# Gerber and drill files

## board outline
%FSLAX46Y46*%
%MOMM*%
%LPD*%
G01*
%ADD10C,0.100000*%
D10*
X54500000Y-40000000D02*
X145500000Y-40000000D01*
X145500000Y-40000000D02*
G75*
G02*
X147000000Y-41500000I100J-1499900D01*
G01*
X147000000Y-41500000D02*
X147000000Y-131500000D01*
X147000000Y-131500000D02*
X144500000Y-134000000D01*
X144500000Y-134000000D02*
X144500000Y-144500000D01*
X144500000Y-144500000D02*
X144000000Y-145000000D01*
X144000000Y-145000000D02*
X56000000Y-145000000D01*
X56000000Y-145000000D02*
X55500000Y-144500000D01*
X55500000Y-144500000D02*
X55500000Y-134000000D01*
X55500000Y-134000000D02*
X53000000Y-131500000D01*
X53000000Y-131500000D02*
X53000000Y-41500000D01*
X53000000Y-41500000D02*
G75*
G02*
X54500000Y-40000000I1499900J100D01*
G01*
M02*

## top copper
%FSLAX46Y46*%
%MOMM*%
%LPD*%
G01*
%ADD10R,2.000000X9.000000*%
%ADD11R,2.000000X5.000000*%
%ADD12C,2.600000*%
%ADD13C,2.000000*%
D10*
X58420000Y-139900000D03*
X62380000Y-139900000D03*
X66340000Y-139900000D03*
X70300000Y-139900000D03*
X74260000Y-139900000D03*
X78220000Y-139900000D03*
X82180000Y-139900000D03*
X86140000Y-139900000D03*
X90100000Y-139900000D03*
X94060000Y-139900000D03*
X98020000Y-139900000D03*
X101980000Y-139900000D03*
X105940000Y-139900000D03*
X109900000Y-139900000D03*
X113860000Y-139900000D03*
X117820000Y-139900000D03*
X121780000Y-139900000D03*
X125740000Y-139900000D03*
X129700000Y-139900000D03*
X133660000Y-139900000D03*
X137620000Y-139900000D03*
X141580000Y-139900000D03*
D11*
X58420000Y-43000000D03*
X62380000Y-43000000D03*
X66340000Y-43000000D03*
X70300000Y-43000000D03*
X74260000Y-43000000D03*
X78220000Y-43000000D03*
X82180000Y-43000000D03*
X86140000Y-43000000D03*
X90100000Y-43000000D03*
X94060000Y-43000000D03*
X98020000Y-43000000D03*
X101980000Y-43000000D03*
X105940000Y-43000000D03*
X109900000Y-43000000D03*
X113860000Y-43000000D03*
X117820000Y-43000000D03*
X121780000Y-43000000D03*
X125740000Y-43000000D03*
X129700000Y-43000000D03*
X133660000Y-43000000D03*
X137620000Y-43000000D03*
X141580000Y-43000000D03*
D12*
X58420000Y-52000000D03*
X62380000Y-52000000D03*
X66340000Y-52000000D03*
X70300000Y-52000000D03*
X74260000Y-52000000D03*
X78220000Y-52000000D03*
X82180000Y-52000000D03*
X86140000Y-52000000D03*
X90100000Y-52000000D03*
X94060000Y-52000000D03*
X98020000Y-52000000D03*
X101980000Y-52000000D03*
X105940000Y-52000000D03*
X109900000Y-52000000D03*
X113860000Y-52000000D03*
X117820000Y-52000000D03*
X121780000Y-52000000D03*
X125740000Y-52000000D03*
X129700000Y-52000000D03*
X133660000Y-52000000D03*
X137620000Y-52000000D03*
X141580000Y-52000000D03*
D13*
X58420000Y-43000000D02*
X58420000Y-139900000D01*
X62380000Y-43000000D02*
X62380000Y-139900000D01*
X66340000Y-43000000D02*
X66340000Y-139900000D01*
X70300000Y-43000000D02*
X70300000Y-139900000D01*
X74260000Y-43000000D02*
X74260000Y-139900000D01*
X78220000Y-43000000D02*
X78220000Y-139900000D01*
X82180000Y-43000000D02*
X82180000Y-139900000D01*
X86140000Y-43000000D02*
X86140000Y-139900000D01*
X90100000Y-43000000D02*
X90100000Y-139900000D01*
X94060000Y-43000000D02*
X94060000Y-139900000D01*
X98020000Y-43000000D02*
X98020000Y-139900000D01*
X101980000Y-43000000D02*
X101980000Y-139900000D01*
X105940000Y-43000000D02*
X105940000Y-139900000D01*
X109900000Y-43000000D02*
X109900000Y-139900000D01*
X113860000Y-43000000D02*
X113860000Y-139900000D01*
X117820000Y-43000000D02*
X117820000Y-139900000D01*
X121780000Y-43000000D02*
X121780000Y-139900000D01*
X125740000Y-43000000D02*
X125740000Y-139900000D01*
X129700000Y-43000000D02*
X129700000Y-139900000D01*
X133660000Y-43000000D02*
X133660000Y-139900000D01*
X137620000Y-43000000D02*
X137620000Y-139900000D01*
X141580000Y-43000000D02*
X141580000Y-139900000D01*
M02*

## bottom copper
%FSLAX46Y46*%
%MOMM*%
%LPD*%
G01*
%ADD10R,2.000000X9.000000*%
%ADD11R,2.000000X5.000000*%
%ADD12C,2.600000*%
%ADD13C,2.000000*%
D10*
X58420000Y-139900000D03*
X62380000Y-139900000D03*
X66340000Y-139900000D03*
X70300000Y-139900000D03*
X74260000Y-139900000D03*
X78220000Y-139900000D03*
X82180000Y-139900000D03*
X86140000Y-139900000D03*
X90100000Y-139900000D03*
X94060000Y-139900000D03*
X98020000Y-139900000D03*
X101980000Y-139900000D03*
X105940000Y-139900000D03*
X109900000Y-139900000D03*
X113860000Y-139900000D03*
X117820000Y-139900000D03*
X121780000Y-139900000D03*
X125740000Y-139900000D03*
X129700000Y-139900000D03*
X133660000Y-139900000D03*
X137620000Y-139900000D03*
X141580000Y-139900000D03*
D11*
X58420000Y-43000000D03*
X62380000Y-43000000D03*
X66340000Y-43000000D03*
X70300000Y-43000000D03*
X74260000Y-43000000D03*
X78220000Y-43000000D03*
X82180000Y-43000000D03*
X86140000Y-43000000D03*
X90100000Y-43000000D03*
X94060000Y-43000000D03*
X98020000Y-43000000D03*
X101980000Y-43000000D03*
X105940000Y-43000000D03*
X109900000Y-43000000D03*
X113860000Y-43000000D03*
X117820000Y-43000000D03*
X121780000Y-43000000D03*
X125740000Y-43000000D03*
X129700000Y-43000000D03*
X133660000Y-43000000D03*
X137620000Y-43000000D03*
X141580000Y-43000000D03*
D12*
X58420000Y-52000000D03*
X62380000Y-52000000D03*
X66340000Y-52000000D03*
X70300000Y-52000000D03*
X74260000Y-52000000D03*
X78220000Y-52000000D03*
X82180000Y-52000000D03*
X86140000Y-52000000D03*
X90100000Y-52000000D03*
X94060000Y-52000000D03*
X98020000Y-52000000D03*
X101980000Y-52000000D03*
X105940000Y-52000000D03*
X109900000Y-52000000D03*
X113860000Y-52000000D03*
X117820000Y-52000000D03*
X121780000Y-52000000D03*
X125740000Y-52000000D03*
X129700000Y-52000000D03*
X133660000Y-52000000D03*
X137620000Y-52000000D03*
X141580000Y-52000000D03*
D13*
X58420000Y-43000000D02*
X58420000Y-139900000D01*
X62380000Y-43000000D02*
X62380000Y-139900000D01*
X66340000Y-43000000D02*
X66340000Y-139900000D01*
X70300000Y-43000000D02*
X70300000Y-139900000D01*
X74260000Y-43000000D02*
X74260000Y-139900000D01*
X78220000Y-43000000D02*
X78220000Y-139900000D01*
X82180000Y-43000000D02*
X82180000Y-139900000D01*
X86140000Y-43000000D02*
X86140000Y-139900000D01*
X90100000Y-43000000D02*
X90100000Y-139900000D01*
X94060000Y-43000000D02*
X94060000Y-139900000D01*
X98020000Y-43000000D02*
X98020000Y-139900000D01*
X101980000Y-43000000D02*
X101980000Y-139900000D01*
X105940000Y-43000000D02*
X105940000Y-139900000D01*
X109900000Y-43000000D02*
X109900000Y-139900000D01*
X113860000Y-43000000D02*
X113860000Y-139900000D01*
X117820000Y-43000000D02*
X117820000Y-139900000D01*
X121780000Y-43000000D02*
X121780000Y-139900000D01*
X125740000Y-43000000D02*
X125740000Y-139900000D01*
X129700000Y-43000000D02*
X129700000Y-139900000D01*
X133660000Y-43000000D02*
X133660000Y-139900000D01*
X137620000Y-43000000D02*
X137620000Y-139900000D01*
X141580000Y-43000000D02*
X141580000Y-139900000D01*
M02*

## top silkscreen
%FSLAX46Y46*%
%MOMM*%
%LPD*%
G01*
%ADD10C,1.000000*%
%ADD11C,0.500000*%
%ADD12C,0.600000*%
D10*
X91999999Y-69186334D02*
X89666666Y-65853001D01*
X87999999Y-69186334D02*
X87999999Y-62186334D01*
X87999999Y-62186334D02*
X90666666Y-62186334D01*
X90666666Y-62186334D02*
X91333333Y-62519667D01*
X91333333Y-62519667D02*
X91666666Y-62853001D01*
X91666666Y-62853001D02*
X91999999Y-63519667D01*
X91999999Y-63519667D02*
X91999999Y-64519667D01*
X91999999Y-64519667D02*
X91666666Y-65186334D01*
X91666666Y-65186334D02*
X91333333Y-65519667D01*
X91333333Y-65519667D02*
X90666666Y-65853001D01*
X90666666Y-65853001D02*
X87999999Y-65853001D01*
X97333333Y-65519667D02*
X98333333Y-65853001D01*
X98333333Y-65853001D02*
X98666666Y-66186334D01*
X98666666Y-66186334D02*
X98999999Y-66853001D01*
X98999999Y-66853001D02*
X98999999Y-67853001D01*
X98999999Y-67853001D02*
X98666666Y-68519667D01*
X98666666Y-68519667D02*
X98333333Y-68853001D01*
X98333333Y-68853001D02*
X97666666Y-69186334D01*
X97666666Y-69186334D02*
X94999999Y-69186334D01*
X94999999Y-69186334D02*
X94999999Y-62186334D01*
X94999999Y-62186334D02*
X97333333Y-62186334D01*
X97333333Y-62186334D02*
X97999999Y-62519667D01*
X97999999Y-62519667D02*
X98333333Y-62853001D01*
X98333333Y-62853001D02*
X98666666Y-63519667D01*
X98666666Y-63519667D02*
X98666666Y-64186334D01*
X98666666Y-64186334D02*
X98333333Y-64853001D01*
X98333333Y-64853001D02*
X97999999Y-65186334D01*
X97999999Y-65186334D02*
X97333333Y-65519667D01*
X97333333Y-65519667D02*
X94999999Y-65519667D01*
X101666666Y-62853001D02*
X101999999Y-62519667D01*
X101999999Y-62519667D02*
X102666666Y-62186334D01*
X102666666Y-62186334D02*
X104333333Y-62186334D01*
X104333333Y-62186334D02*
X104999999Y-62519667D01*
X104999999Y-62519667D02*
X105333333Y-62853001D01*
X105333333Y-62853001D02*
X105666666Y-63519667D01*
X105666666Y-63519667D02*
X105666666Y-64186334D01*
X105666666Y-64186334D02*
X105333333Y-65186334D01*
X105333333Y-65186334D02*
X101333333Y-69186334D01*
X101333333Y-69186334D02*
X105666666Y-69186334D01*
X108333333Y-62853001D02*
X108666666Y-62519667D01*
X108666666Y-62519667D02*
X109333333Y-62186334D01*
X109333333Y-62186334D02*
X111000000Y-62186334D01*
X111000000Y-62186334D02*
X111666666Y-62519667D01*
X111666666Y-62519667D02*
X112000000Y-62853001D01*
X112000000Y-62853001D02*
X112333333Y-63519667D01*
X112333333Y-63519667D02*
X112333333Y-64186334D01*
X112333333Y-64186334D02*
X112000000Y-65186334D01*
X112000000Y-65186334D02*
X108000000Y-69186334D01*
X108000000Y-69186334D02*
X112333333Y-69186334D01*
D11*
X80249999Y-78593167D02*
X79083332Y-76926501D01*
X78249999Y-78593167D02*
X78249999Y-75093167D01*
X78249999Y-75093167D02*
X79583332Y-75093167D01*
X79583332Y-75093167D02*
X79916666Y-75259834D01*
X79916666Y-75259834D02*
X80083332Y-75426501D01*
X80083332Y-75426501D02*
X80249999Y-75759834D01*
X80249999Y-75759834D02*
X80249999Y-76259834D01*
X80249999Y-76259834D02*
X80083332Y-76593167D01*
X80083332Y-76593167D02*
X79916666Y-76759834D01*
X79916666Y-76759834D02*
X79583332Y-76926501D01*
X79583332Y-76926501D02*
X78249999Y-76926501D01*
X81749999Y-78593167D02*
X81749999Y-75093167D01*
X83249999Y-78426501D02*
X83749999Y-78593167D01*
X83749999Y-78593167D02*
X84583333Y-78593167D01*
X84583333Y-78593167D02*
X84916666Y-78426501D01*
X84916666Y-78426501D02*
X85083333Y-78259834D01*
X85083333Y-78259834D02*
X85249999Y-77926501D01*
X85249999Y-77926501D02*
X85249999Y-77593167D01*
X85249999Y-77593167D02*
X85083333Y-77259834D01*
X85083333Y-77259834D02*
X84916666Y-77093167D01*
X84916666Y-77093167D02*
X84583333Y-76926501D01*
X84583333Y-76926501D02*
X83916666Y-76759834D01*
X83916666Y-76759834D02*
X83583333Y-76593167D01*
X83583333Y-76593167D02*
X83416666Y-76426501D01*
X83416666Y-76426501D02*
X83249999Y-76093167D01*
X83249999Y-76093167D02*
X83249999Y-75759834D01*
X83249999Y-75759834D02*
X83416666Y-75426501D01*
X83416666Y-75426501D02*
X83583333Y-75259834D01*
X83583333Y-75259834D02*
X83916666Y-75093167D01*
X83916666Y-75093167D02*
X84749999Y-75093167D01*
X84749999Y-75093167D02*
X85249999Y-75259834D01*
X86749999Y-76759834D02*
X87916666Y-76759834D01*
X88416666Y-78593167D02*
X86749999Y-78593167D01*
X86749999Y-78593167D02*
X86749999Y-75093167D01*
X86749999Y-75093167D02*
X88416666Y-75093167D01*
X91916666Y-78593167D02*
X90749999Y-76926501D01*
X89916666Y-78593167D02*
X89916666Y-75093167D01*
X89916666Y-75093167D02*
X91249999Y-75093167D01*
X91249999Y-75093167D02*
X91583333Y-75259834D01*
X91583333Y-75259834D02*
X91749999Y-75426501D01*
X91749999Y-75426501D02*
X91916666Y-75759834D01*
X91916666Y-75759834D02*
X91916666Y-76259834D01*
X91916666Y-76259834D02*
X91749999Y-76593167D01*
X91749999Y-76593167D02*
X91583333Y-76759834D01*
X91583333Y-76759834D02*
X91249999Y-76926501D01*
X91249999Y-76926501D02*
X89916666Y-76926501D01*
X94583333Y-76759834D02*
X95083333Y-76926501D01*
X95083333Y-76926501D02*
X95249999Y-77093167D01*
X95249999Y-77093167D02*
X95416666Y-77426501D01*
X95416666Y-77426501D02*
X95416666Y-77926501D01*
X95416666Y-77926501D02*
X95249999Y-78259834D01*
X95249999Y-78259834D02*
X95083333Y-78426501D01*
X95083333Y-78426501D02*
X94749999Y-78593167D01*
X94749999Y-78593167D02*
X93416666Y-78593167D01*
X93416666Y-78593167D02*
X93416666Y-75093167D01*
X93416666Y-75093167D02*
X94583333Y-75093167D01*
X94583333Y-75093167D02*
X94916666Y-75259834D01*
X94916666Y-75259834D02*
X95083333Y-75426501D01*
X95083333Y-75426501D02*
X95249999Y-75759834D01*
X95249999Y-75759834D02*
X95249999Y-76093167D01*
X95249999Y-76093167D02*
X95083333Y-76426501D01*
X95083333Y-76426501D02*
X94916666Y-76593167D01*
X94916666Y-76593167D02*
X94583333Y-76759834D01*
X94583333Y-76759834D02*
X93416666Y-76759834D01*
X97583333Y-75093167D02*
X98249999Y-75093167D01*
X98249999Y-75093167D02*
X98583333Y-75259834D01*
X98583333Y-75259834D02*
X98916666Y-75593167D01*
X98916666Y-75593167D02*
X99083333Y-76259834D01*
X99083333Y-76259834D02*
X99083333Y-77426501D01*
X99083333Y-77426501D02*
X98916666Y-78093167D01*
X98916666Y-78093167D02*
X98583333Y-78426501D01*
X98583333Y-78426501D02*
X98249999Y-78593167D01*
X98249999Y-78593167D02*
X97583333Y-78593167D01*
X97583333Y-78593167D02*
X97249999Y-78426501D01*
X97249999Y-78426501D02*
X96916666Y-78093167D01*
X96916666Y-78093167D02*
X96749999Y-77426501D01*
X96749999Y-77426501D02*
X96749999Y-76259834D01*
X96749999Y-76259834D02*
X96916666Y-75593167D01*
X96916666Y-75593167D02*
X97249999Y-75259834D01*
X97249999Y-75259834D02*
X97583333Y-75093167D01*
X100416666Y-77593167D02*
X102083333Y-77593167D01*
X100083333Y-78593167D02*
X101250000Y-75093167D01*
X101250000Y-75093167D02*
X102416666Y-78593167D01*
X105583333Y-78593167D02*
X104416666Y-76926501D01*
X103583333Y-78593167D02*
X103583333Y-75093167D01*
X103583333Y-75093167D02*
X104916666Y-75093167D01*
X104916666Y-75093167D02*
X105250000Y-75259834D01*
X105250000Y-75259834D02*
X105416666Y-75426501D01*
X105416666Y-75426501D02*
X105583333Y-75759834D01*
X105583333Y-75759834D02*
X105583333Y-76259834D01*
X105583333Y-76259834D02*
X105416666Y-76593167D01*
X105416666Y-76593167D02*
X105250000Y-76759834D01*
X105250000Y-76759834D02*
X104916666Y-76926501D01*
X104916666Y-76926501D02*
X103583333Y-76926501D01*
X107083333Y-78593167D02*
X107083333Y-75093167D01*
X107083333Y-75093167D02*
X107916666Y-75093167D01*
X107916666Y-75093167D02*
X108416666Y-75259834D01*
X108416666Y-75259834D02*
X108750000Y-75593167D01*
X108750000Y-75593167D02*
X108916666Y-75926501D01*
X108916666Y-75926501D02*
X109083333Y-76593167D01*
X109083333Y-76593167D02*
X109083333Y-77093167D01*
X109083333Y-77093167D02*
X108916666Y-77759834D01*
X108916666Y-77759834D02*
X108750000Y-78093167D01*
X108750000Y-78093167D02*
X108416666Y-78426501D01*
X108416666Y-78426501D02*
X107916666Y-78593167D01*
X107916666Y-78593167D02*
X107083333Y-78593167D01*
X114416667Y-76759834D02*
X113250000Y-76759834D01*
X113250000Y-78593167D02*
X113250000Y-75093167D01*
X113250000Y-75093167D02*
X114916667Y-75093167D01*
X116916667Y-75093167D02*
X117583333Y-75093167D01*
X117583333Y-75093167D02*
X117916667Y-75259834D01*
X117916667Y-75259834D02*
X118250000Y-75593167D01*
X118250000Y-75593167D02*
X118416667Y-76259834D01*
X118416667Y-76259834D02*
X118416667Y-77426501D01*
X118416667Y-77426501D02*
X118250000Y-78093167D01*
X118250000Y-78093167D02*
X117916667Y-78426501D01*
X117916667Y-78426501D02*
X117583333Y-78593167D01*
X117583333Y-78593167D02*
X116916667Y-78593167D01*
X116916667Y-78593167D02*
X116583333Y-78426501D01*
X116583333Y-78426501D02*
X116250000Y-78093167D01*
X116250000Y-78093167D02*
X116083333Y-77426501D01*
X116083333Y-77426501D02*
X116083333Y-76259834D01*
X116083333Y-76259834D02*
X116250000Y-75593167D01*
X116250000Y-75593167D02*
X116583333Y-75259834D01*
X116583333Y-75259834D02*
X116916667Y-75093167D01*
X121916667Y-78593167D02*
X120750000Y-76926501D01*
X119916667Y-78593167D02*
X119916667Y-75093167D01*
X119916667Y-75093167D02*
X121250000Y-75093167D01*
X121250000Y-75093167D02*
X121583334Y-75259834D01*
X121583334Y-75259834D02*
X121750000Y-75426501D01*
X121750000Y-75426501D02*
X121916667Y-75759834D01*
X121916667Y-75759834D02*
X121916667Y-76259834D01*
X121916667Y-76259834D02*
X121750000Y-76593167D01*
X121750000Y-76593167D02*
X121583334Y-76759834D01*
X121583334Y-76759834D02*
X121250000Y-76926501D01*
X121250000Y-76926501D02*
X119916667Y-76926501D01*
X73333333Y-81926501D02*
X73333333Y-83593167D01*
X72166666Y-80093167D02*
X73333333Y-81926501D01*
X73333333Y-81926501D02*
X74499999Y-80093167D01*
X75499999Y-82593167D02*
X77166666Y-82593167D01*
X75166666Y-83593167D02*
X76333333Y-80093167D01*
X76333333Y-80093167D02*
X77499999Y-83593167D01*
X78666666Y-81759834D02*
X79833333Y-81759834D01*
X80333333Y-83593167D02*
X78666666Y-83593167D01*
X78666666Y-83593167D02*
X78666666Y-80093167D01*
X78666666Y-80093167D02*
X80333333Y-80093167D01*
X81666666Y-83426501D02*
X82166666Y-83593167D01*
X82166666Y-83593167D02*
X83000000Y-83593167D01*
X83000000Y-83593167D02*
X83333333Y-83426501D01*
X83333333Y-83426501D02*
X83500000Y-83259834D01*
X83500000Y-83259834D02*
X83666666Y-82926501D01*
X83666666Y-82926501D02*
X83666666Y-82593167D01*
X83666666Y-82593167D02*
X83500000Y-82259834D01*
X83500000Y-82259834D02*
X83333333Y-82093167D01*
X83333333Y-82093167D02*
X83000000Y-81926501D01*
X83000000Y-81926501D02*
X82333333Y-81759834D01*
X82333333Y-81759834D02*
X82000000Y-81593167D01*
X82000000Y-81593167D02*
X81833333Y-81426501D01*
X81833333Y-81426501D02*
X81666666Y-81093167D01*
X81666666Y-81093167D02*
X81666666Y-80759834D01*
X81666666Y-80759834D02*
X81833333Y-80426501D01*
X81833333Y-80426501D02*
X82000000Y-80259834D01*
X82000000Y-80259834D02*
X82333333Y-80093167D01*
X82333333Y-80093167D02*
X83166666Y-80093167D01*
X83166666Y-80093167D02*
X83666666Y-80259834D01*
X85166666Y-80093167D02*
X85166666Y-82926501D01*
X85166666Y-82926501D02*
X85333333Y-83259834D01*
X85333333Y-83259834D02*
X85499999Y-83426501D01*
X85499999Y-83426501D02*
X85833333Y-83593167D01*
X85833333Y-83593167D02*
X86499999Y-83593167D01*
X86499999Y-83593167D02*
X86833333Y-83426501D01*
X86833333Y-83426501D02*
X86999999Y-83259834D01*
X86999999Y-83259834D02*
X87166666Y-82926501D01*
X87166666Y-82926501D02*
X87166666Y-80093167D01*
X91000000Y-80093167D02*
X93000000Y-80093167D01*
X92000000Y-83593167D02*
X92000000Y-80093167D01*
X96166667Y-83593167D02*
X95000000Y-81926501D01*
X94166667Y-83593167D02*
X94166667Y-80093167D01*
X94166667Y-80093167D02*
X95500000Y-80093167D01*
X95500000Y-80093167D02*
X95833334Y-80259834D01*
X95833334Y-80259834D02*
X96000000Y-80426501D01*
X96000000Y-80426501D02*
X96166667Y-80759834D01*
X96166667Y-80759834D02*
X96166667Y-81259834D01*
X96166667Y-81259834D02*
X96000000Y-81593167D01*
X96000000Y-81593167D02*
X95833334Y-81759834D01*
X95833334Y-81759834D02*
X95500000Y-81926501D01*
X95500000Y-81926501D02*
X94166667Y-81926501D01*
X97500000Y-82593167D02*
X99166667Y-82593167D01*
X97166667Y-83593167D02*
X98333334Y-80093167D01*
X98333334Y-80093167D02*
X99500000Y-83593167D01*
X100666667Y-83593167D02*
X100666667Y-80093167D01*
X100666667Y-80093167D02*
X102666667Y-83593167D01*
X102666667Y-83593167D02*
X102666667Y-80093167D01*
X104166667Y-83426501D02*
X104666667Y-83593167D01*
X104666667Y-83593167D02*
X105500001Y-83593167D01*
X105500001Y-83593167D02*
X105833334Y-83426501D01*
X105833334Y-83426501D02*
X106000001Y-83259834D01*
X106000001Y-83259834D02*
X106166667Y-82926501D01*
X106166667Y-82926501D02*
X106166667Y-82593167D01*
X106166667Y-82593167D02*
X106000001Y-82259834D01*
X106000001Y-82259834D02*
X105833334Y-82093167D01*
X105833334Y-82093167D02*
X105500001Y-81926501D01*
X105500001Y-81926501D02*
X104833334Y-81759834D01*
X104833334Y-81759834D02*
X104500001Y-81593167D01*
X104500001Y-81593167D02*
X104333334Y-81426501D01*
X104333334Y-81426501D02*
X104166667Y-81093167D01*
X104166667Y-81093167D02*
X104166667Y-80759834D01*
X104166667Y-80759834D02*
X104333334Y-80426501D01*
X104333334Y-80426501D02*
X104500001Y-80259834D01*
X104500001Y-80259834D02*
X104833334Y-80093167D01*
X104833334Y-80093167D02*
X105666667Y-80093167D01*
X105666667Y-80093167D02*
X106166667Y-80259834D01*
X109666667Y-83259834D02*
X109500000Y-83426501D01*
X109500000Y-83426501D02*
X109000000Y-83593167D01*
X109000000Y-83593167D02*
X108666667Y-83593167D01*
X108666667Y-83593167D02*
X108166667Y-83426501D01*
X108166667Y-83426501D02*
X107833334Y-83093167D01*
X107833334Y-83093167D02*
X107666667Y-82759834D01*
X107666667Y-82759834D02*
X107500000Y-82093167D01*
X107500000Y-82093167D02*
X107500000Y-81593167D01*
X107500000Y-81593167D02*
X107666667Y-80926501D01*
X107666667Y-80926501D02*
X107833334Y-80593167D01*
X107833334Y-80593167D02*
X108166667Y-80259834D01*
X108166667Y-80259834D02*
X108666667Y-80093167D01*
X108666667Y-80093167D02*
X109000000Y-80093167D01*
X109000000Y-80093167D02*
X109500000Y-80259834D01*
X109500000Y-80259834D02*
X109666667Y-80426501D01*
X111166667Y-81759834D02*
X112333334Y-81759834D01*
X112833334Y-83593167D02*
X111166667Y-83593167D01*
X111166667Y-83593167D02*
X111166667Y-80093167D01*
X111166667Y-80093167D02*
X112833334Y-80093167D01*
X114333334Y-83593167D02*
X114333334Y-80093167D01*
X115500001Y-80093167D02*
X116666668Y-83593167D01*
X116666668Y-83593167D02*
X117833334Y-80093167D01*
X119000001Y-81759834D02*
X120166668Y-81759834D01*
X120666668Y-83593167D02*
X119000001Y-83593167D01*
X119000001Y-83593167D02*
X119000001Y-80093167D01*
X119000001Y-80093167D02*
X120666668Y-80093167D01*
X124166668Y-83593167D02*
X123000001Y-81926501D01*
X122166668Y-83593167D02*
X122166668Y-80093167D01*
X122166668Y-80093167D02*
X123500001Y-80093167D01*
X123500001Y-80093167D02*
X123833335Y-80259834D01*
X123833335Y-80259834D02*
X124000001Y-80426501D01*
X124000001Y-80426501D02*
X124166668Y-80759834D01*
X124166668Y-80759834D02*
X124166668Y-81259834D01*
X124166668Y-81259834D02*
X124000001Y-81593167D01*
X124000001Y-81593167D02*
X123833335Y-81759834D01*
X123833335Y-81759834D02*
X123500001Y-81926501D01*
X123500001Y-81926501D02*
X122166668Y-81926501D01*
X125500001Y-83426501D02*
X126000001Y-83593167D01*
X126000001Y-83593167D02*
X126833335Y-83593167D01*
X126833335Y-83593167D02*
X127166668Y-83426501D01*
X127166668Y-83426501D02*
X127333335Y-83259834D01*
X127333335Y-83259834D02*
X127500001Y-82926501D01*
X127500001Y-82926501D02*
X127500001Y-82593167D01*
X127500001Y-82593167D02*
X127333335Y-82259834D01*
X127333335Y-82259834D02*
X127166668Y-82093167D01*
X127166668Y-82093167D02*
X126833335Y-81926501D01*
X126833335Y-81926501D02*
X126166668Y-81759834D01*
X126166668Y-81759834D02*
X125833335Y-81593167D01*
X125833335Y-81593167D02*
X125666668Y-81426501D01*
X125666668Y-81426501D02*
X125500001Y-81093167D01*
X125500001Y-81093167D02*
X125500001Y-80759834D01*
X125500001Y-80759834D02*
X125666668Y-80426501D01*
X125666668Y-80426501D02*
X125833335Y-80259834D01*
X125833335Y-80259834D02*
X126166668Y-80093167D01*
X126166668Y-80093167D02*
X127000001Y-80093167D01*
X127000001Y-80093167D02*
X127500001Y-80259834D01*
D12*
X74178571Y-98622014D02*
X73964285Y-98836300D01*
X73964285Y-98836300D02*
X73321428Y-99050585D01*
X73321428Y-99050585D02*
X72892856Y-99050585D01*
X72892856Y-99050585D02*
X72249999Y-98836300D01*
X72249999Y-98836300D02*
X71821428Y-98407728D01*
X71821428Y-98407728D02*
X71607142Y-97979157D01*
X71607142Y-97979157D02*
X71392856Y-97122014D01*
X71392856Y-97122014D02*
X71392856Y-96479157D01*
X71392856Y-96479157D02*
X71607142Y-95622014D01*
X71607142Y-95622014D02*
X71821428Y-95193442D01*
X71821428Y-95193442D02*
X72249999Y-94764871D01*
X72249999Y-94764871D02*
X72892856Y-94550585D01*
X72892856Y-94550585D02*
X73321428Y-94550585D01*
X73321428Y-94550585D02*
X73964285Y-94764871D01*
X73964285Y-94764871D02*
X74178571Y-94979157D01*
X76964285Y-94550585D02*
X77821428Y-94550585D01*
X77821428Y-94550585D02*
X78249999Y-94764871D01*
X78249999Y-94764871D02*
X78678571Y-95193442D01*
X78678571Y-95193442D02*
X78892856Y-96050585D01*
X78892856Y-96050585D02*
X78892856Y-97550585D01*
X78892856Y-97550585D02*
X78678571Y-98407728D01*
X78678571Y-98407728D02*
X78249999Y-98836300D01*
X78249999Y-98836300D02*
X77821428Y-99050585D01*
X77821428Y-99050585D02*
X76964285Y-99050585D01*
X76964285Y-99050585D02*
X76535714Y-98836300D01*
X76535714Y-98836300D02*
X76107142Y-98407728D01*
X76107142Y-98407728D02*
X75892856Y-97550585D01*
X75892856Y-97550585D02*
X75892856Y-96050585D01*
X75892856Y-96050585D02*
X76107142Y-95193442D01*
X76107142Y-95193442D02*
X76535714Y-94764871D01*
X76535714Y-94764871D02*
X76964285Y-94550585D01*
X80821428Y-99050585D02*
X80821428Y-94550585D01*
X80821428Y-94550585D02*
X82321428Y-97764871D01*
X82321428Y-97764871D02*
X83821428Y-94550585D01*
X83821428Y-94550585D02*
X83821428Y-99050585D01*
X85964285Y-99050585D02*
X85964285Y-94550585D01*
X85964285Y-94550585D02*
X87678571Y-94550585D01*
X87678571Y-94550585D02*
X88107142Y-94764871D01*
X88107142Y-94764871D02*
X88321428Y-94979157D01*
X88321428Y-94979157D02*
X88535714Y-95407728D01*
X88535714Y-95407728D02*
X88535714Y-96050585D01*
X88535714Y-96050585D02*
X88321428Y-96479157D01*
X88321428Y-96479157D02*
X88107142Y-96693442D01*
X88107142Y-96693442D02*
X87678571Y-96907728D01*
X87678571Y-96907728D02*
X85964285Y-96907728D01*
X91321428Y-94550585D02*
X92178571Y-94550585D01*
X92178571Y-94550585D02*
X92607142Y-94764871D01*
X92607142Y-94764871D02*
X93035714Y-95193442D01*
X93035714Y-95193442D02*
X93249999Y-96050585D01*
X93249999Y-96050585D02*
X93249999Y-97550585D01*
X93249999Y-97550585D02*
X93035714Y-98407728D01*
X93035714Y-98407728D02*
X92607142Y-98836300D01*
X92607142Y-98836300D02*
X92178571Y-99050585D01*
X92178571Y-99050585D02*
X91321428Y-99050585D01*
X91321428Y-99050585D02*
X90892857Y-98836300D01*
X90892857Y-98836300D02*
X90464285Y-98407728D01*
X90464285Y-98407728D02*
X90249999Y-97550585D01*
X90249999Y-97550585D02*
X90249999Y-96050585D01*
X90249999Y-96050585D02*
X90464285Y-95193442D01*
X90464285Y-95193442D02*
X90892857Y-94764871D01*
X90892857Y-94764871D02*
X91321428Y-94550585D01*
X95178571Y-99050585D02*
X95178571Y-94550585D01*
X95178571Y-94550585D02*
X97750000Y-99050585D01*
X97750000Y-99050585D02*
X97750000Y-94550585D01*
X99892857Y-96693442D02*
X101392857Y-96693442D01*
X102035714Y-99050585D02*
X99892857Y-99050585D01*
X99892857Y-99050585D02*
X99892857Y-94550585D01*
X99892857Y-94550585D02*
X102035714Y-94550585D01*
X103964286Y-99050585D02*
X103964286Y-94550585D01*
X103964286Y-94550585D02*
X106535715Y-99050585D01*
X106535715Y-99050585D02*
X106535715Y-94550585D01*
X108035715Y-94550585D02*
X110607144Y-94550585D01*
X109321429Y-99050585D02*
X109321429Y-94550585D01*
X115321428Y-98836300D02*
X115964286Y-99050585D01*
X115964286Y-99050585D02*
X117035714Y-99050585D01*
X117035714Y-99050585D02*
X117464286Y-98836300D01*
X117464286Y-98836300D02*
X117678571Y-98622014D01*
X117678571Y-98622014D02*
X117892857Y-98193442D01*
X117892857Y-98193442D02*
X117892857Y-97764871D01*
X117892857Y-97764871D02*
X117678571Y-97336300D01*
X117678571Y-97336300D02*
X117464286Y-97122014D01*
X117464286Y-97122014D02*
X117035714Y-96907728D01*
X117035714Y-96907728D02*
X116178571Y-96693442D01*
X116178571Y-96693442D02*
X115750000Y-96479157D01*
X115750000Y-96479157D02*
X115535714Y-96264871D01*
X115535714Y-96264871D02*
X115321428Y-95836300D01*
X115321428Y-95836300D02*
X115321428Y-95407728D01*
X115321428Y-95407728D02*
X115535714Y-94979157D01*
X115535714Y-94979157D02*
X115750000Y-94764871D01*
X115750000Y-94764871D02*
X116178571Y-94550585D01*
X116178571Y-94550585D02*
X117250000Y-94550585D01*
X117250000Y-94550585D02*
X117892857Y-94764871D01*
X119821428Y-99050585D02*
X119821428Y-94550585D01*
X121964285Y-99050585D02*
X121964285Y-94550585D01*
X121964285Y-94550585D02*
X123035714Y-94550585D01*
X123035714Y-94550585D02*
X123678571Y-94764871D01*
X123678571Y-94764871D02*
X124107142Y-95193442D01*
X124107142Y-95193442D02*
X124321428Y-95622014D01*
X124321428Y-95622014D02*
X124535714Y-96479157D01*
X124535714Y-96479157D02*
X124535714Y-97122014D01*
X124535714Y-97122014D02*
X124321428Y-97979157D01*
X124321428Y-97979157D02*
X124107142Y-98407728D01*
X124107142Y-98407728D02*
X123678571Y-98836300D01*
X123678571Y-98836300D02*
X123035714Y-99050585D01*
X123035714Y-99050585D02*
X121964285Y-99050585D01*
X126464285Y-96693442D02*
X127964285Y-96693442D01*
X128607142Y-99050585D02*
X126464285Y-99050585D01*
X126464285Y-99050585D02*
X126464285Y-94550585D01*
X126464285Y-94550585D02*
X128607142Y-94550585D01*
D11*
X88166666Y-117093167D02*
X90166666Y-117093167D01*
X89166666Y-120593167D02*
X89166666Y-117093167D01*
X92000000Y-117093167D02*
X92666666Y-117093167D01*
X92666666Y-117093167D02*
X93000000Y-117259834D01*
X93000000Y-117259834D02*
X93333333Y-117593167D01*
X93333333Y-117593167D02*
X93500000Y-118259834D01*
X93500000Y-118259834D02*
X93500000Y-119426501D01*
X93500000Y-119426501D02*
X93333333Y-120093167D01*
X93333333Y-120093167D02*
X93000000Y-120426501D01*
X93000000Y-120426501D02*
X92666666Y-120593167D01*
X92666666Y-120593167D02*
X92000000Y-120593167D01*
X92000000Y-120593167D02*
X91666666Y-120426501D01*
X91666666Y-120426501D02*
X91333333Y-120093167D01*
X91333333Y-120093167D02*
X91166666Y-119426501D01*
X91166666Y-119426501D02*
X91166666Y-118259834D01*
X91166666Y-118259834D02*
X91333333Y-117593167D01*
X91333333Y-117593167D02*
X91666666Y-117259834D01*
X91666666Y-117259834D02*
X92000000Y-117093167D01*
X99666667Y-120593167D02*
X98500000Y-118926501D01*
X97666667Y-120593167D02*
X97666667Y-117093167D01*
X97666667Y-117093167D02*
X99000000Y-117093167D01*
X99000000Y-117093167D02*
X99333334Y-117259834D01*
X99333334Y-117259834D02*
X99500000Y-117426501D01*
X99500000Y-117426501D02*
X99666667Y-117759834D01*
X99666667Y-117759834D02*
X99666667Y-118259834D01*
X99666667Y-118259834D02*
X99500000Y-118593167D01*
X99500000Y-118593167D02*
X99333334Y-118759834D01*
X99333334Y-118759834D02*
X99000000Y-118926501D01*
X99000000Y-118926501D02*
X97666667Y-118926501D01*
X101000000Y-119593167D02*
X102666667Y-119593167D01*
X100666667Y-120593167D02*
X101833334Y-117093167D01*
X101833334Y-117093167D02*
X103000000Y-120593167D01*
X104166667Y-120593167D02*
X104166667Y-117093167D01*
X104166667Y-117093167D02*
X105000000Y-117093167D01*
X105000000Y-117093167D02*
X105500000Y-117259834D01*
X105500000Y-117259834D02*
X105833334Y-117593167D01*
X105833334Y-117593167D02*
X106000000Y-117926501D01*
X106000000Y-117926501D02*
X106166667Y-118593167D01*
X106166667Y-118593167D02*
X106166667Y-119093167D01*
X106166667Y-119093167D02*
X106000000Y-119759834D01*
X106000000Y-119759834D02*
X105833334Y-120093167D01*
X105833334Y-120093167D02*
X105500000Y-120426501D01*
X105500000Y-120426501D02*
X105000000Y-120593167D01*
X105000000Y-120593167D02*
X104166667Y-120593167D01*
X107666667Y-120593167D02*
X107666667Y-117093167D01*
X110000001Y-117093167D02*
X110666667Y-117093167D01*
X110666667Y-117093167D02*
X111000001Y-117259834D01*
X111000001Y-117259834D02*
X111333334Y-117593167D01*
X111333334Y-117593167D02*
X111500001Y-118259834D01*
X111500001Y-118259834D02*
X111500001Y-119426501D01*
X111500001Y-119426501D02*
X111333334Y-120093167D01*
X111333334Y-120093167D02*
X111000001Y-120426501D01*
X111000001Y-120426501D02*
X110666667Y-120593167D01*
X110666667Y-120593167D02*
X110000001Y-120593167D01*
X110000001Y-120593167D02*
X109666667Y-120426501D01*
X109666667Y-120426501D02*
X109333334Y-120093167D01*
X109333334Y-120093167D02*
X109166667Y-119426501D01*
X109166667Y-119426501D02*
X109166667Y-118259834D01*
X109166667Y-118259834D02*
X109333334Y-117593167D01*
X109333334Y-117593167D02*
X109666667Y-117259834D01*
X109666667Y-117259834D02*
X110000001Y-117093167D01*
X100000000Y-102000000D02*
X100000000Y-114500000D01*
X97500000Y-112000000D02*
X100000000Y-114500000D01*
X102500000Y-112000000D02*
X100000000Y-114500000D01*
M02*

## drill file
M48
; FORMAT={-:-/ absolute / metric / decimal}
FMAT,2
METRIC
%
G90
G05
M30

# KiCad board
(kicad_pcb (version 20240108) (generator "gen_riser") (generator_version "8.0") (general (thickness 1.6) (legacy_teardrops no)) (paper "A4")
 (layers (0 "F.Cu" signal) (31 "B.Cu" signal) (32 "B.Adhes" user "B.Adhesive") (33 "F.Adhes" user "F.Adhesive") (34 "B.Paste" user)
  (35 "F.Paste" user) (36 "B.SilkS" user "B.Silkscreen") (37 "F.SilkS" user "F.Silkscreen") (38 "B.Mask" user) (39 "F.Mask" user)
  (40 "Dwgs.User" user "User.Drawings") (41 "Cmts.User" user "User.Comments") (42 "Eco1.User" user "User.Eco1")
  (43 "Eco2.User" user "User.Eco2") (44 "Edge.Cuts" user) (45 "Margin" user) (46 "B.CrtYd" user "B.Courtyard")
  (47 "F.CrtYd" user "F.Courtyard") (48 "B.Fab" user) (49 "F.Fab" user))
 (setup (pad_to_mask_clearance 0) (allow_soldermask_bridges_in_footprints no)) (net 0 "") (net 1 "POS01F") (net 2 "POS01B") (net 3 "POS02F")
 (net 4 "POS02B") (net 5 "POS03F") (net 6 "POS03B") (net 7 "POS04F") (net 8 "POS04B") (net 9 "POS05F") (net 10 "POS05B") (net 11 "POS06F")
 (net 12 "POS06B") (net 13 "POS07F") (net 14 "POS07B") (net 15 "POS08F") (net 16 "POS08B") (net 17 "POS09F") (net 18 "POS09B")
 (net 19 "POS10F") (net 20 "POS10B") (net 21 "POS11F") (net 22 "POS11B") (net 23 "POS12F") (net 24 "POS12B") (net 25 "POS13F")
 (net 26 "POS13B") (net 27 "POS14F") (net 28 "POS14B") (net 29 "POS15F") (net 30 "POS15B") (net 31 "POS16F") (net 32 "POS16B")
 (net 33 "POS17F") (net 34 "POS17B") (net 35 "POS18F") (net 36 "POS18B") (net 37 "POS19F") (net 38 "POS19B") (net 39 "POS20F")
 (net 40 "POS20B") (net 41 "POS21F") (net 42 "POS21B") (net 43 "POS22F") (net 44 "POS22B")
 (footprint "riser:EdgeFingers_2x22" (layer "F.Cu") (at 100 40)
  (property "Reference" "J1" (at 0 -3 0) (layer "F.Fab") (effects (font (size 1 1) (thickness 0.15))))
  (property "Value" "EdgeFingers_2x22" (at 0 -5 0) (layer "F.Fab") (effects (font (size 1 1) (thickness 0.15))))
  (pad "1" smd rect (at -41.58 99.9) (size 2 9) (layers "F.Cu" "F.Mask") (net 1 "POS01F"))
  (pad "1B" smd rect (at -41.58 99.9) (size 2 9) (layers "B.Cu" "B.Mask") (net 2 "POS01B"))
  (pad "2" smd rect (at -37.62 99.9) (size 2 9) (layers "F.Cu" "F.Mask") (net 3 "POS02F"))
  (pad "2B" smd rect (at -37.62 99.9) (size 2 9) (layers "B.Cu" "B.Mask") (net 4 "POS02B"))
  (pad "3" smd rect (at -33.66 99.9) (size 2 9) (layers "F.Cu" "F.Mask") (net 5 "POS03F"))
  (pad "3B" smd rect (at -33.66 99.9) (size 2 9) (layers "B.Cu" "B.Mask") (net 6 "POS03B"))
  (pad "4" smd rect (at -29.7 99.9) (size 2 9) (layers "F.Cu" "F.Mask") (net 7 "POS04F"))
  (pad "4B" smd rect (at -29.7 99.9) (size 2 9) (layers "B.Cu" "B.Mask") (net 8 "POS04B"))
  (pad "5" smd rect (at -25.74 99.9) (size 2 9) (layers "F.Cu" "F.Mask") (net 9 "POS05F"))
  (pad "5B" smd rect (at -25.74 99.9) (size 2 9) (layers "B.Cu" "B.Mask") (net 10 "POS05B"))
  (pad "6" smd rect (at -21.78 99.9) (size 2 9) (layers "F.Cu" "F.Mask") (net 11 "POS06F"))
  (pad "6B" smd rect (at -21.78 99.9) (size 2 9) (layers "B.Cu" "B.Mask") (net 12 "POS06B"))
  (pad "7" smd rect (at -17.82 99.9) (size 2 9) (layers "F.Cu" "F.Mask") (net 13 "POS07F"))
  (pad "7B" smd rect (at -17.82 99.9) (size 2 9) (layers "B.Cu" "B.Mask") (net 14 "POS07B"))
  (pad "8" smd rect (at -13.86 99.9) (size 2 9) (layers "F.Cu" "F.Mask") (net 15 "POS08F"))
  (pad "8B" smd rect (at -13.86 99.9) (size 2 9) (layers "B.Cu" "B.Mask") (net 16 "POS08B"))
  (pad "9" smd rect (at -9.9 99.9) (size 2 9) (layers "F.Cu" "F.Mask") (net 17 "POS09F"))
  (pad "9B" smd rect (at -9.9 99.9) (size 2 9) (layers "B.Cu" "B.Mask") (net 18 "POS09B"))
  (pad "10" smd rect (at -5.94 99.9) (size 2 9) (layers "F.Cu" "F.Mask") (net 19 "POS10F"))
  (pad "10B" smd rect (at -5.94 99.9) (size 2 9) (layers "B.Cu" "B.Mask") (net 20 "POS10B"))
  (pad "11" smd rect (at -1.98 99.9) (size 2 9) (layers "F.Cu" "F.Mask") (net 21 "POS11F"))
  (pad "11B" smd rect (at -1.98 99.9) (size 2 9) (layers "B.Cu" "B.Mask") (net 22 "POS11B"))
  (pad "12" smd rect (at 1.98 99.9) (size 2 9) (layers "F.Cu" "F.Mask") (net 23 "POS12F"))
  (pad "12B" smd rect (at 1.98 99.9) (size 2 9) (layers "B.Cu" "B.Mask") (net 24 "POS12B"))
  (pad "13" smd rect (at 5.94 99.9) (size 2 9) (layers "F.Cu" "F.Mask") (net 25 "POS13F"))
  (pad "13B" smd rect (at 5.94 99.9) (size 2 9) (layers "B.Cu" "B.Mask") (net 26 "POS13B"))
  (pad "14" smd rect (at 9.9 99.9) (size 2 9) (layers "F.Cu" "F.Mask") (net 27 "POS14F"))
  (pad "14B" smd rect (at 9.9 99.9) (size 2 9) (layers "B.Cu" "B.Mask") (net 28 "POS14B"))
  (pad "15" smd rect (at 13.86 99.9) (size 2 9) (layers "F.Cu" "F.Mask") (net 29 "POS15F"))
  (pad "15B" smd rect (at 13.86 99.9) (size 2 9) (layers "B.Cu" "B.Mask") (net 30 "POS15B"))
  (pad "16" smd rect (at 17.82 99.9) (size 2 9) (layers "F.Cu" "F.Mask") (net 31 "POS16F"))
  (pad "16B" smd rect (at 17.82 99.9) (size 2 9) (layers "B.Cu" "B.Mask") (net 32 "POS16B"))
  (pad "17" smd rect (at 21.78 99.9) (size 2 9) (layers "F.Cu" "F.Mask") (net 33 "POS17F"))
  (pad "17B" smd rect (at 21.78 99.9) (size 2 9) (layers "B.Cu" "B.Mask") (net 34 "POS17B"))
  (pad "18" smd rect (at 25.74 99.9) (size 2 9) (layers "F.Cu" "F.Mask") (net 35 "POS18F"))
  (pad "18B" smd rect (at 25.74 99.9) (size 2 9) (layers "B.Cu" "B.Mask") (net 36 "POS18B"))
  (pad "19" smd rect (at 29.7 99.9) (size 2 9) (layers "F.Cu" "F.Mask") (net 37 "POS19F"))
  (pad "19B" smd rect (at 29.7 99.9) (size 2 9) (layers "B.Cu" "B.Mask") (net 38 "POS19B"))
  (pad "20" smd rect (at 33.66 99.9) (size 2 9) (layers "F.Cu" "F.Mask") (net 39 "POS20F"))
  (pad "20B" smd rect (at 33.66 99.9) (size 2 9) (layers "B.Cu" "B.Mask") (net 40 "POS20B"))
  (pad "21" smd rect (at 37.62 99.9) (size 2 9) (layers "F.Cu" "F.Mask") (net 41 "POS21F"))
  (pad "21B" smd rect (at 37.62 99.9) (size 2 9) (layers "B.Cu" "B.Mask") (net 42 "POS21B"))
  (pad "22" smd rect (at 41.58 99.9) (size 2 9) (layers "F.Cu" "F.Mask") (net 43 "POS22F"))
  (pad "22B" smd rect (at 41.58 99.9) (size 2 9) (layers "B.Cu" "B.Mask") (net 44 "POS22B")))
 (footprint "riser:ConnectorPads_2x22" (layer "F.Cu") (at 100 40)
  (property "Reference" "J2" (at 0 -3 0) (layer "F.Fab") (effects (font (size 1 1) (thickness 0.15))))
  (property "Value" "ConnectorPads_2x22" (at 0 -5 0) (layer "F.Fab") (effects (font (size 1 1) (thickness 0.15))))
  (pad "1" smd rect (at -41.58 3) (size 2 5) (layers "F.Cu" "F.Mask") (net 1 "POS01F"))
  (pad "1B" smd rect (at -41.58 3) (size 2 5) (layers "B.Cu" "B.Mask") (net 2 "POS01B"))
  (pad "2" smd rect (at -37.62 3) (size 2 5) (layers "F.Cu" "F.Mask") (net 3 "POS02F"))
  (pad "2B" smd rect (at -37.62 3) (size 2 5) (layers "B.Cu" "B.Mask") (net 4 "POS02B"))
  (pad "3" smd rect (at -33.66 3) (size 2 5) (layers "F.Cu" "F.Mask") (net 5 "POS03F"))
  (pad "3B" smd rect (at -33.66 3) (size 2 5) (layers "B.Cu" "B.Mask") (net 6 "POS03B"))
  (pad "4" smd rect (at -29.7 3) (size 2 5) (layers "F.Cu" "F.Mask") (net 7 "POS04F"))
  (pad "4B" smd rect (at -29.7 3) (size 2 5) (layers "B.Cu" "B.Mask") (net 8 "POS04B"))
  (pad "5" smd rect (at -25.74 3) (size 2 5) (layers "F.Cu" "F.Mask") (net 9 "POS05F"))
  (pad "5B" smd rect (at -25.74 3) (size 2 5) (layers "B.Cu" "B.Mask") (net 10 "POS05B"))
  (pad "6" smd rect (at -21.78 3) (size 2 5) (layers "F.Cu" "F.Mask") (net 11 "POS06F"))
  (pad "6B" smd rect (at -21.78 3) (size 2 5) (layers "B.Cu" "B.Mask") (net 12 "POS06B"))
  (pad "7" smd rect (at -17.82 3) (size 2 5) (layers "F.Cu" "F.Mask") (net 13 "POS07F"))
  (pad "7B" smd rect (at -17.82 3) (size 2 5) (layers "B.Cu" "B.Mask") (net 14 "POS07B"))
  (pad "8" smd rect (at -13.86 3) (size 2 5) (layers "F.Cu" "F.Mask") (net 15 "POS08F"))
  (pad "8B" smd rect (at -13.86 3) (size 2 5) (layers "B.Cu" "B.Mask") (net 16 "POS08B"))
  (pad "9" smd rect (at -9.9 3) (size 2 5) (layers "F.Cu" "F.Mask") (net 17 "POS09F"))
  (pad "9B" smd rect (at -9.9 3) (size 2 5) (layers "B.Cu" "B.Mask") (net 18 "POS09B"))
  (pad "10" smd rect (at -5.94 3) (size 2 5) (layers "F.Cu" "F.Mask") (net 19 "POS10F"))
  (pad "10B" smd rect (at -5.94 3) (size 2 5) (layers "B.Cu" "B.Mask") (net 20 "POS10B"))
  (pad "11" smd rect (at -1.98 3) (size 2 5) (layers "F.Cu" "F.Mask") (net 21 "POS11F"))
  (pad "11B" smd rect (at -1.98 3) (size 2 5) (layers "B.Cu" "B.Mask") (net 22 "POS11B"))
  (pad "12" smd rect (at 1.98 3) (size 2 5) (layers "F.Cu" "F.Mask") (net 23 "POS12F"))
  (pad "12B" smd rect (at 1.98 3) (size 2 5) (layers "B.Cu" "B.Mask") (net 24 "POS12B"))
  (pad "13" smd rect (at 5.94 3) (size 2 5) (layers "F.Cu" "F.Mask") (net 25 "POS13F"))
  (pad "13B" smd rect (at 5.94 3) (size 2 5) (layers "B.Cu" "B.Mask") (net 26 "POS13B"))
  (pad "14" smd rect (at 9.9 3) (size 2 5) (layers "F.Cu" "F.Mask") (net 27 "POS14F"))
  (pad "14B" smd rect (at 9.9 3) (size 2 5) (layers "B.Cu" "B.Mask") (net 28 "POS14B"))
  (pad "15" smd rect (at 13.86 3) (size 2 5) (layers "F.Cu" "F.Mask") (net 29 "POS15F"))
  (pad "15B" smd rect (at 13.86 3) (size 2 5) (layers "B.Cu" "B.Mask") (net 30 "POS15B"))
  (pad "16" smd rect (at 17.82 3) (size 2 5) (layers "F.Cu" "F.Mask") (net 31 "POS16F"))
  (pad "16B" smd rect (at 17.82 3) (size 2 5) (layers "B.Cu" "B.Mask") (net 32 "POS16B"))
  (pad "17" smd rect (at 21.78 3) (size 2 5) (layers "F.Cu" "F.Mask") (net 33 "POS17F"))
  (pad "17B" smd rect (at 21.78 3) (size 2 5) (layers "B.Cu" "B.Mask") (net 34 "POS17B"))
  (pad "18" smd rect (at 25.74 3) (size 2 5) (layers "F.Cu" "F.Mask") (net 35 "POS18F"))
  (pad "18B" smd rect (at 25.74 3) (size 2 5) (layers "B.Cu" "B.Mask") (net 36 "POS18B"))
  (pad "19" smd rect (at 29.7 3) (size 2 5) (layers "F.Cu" "F.Mask") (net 37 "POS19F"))
  (pad "19B" smd rect (at 29.7 3) (size 2 5) (layers "B.Cu" "B.Mask") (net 38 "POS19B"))
  (pad "20" smd rect (at 33.66 3) (size 2 5) (layers "F.Cu" "F.Mask") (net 39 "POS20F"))
  (pad "20B" smd rect (at 33.66 3) (size 2 5) (layers "B.Cu" "B.Mask") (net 40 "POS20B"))
  (pad "21" smd rect (at 37.62 3) (size 2 5) (layers "F.Cu" "F.Mask") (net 41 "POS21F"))
  (pad "21B" smd rect (at 37.62 3) (size 2 5) (layers "B.Cu" "B.Mask") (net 42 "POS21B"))
  (pad "22" smd rect (at 41.58 3) (size 2 5) (layers "F.Cu" "F.Mask") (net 43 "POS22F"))
  (pad "22B" smd rect (at 41.58 3) (size 2 5) (layers "B.Cu" "B.Mask") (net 44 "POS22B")))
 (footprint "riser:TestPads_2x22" (layer "F.Cu") (at 100 40)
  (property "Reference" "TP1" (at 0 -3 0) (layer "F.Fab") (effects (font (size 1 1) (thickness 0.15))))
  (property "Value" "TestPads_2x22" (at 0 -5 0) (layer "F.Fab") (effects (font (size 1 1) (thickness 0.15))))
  (pad "1" smd circle (at -41.58 12) (size 2.6 2.6) (layers "F.Cu" "F.Mask") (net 1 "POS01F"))
  (pad "1B" smd circle (at -41.58 12) (size 2.6 2.6) (layers "B.Cu" "B.Mask") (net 2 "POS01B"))
  (pad "2" smd circle (at -37.62 12) (size 2.6 2.6) (layers "F.Cu" "F.Mask") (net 3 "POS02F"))
  (pad "2B" smd circle (at -37.62 12) (size 2.6 2.6) (layers "B.Cu" "B.Mask") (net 4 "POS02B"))
  (pad "3" smd circle (at -33.66 12) (size 2.6 2.6) (layers "F.Cu" "F.Mask") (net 5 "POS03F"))
  (pad "3B" smd circle (at -33.66 12) (size 2.6 2.6) (layers "B.Cu" "B.Mask") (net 6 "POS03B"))
  (pad "4" smd circle (at -29.7 12) (size 2.6 2.6) (layers "F.Cu" "F.Mask") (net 7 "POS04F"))
  (pad "4B" smd circle (at -29.7 12) (size 2.6 2.6) (layers "B.Cu" "B.Mask") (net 8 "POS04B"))
  (pad "5" smd circle (at -25.74 12) (size 2.6 2.6) (layers "F.Cu" "F.Mask") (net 9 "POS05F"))
  (pad "5B" smd circle (at -25.74 12) (size 2.6 2.6) (layers "B.Cu" "B.Mask") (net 10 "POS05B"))
  (pad "6" smd circle (at -21.78 12) (size 2.6 2.6) (layers "F.Cu" "F.Mask") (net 11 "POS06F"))
  (pad "6B" smd circle (at -21.78 12) (size 2.6 2.6) (layers "B.Cu" "B.Mask") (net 12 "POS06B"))
  (pad "7" smd circle (at -17.82 12) (size 2.6 2.6) (layers "F.Cu" "F.Mask") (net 13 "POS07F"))
  (pad "7B" smd circle (at -17.82 12) (size 2.6 2.6) (layers "B.Cu" "B.Mask") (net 14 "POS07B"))
  (pad "8" smd circle (at -13.86 12) (size 2.6 2.6) (layers "F.Cu" "F.Mask") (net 15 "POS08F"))
  (pad "8B" smd circle (at -13.86 12) (size 2.6 2.6) (layers "B.Cu" "B.Mask") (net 16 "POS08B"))
  (pad "9" smd circle (at -9.9 12) (size 2.6 2.6) (layers "F.Cu" "F.Mask") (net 17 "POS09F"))
  (pad "9B" smd circle (at -9.9 12) (size 2.6 2.6) (layers "B.Cu" "B.Mask") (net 18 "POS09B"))
  (pad "10" smd circle (at -5.94 12) (size 2.6 2.6) (layers "F.Cu" "F.Mask") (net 19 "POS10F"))
  (pad "10B" smd circle (at -5.94 12) (size 2.6 2.6) (layers "B.Cu" "B.Mask") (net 20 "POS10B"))
  (pad "11" smd circle (at -1.98 12) (size 2.6 2.6) (layers "F.Cu" "F.Mask") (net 21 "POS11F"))
  (pad "11B" smd circle (at -1.98 12) (size 2.6 2.6) (layers "B.Cu" "B.Mask") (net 22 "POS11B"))
  (pad "12" smd circle (at 1.98 12) (size 2.6 2.6) (layers "F.Cu" "F.Mask") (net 23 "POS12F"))
  (pad "12B" smd circle (at 1.98 12) (size 2.6 2.6) (layers "B.Cu" "B.Mask") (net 24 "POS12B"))
  (pad "13" smd circle (at 5.94 12) (size 2.6 2.6) (layers "F.Cu" "F.Mask") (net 25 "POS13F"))
  (pad "13B" smd circle (at 5.94 12) (size 2.6 2.6) (layers "B.Cu" "B.Mask") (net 26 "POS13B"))
  (pad "14" smd circle (at 9.9 12) (size 2.6 2.6) (layers "F.Cu" "F.Mask") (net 27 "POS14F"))
  (pad "14B" smd circle (at 9.9 12) (size 2.6 2.6) (layers "B.Cu" "B.Mask") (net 28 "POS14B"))
  (pad "15" smd circle (at 13.86 12) (size 2.6 2.6) (layers "F.Cu" "F.Mask") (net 29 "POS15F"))
  (pad "15B" smd circle (at 13.86 12) (size 2.6 2.6) (layers "B.Cu" "B.Mask") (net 30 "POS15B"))
  (pad "16" smd circle (at 17.82 12) (size 2.6 2.6) (layers "F.Cu" "F.Mask") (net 31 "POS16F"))
  (pad "16B" smd circle (at 17.82 12) (size 2.6 2.6) (layers "B.Cu" "B.Mask") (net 32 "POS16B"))
  (pad "17" smd circle (at 21.78 12) (size 2.6 2.6) (layers "F.Cu" "F.Mask") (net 33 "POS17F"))
  (pad "17B" smd circle (at 21.78 12) (size 2.6 2.6) (layers "B.Cu" "B.Mask") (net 34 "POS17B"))
  (pad "18" smd circle (at 25.74 12) (size 2.6 2.6) (layers "F.Cu" "F.Mask") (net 35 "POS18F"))
  (pad "18B" smd circle (at 25.74 12) (size 2.6 2.6) (layers "B.Cu" "B.Mask") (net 36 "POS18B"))
  (pad "19" smd circle (at 29.7 12) (size 2.6 2.6) (layers "F.Cu" "F.Mask") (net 37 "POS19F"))
  (pad "19B" smd circle (at 29.7 12) (size 2.6 2.6) (layers "B.Cu" "B.Mask") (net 38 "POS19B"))
  (pad "20" smd circle (at 33.66 12) (size 2.6 2.6) (layers "F.Cu" "F.Mask") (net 39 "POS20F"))
  (pad "20B" smd circle (at 33.66 12) (size 2.6 2.6) (layers "B.Cu" "B.Mask") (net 40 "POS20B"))
  (pad "21" smd circle (at 37.62 12) (size 2.6 2.6) (layers "F.Cu" "F.Mask") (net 41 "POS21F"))
  (pad "21B" smd circle (at 37.62 12) (size 2.6 2.6) (layers "B.Cu" "B.Mask") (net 42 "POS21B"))
  (pad "22" smd circle (at 41.58 12) (size 2.6 2.6) (layers "F.Cu" "F.Mask") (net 43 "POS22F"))
  (pad "22B" smd circle (at 41.58 12) (size 2.6 2.6) (layers "B.Cu" "B.Mask") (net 44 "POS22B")))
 (segment (start 58.42 43) (end 58.42 139.9) (width 2) (layer "F.Cu") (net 1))
 (segment (start 58.42 43) (end 58.42 139.9) (width 2) (layer "B.Cu") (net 2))
 (segment (start 62.38 43) (end 62.38 139.9) (width 2) (layer "F.Cu") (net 3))
 (segment (start 62.38 43) (end 62.38 139.9) (width 2) (layer "B.Cu") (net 4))
 (segment (start 66.34 43) (end 66.34 139.9) (width 2) (layer "F.Cu") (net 5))
 (segment (start 66.34 43) (end 66.34 139.9) (width 2) (layer "B.Cu") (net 6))
 (segment (start 70.3 43) (end 70.3 139.9) (width 2) (layer "F.Cu") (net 7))
 (segment (start 70.3 43) (end 70.3 139.9) (width 2) (layer "B.Cu") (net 8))
 (segment (start 74.26 43) (end 74.26 139.9) (width 2) (layer "F.Cu") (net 9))
 (segment (start 74.26 43) (end 74.26 139.9) (width 2) (layer "B.Cu") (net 10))
 (segment (start 78.22 43) (end 78.22 139.9) (width 2) (layer "F.Cu") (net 11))
 (segment (start 78.22 43) (end 78.22 139.9) (width 2) (layer "B.Cu") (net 12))
 (segment (start 82.18 43) (end 82.18 139.9) (width 2) (layer "F.Cu") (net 13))
 (segment (start 82.18 43) (end 82.18 139.9) (width 2) (layer "B.Cu") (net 14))
 (segment (start 86.14 43) (end 86.14 139.9) (width 2) (layer "F.Cu") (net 15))
 (segment (start 86.14 43) (end 86.14 139.9) (width 2) (layer "B.Cu") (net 16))
 (segment (start 90.1 43) (end 90.1 139.9) (width 2) (layer "F.Cu") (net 17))
 (segment (start 90.1 43) (end 90.1 139.9) (width 2) (layer "B.Cu") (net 18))
 (segment (start 94.06 43) (end 94.06 139.9) (width 2) (layer "F.Cu") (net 19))
 (segment (start 94.06 43) (end 94.06 139.9) (width 2) (layer "B.Cu") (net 20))
 (segment (start 98.02 43) (end 98.02 139.9) (width 2) (layer "F.Cu") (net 21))
 (segment (start 98.02 43) (end 98.02 139.9) (width 2) (layer "B.Cu") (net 22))
 (segment (start 101.98 43) (end 101.98 139.9) (width 2) (layer "F.Cu") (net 23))
 (segment (start 101.98 43) (end 101.98 139.9) (width 2) (layer "B.Cu") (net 24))
 (segment (start 105.94 43) (end 105.94 139.9) (width 2) (layer "F.Cu") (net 25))
 (segment (start 105.94 43) (end 105.94 139.9) (width 2) (layer "B.Cu") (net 26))
 (segment (start 109.9 43) (end 109.9 139.9) (width 2) (layer "F.Cu") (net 27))
 (segment (start 109.9 43) (end 109.9 139.9) (width 2) (layer "B.Cu") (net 28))
 (segment (start 113.86 43) (end 113.86 139.9) (width 2) (layer "F.Cu") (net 29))
 (segment (start 113.86 43) (end 113.86 139.9) (width 2) (layer "B.Cu") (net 30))
 (segment (start 117.82 43) (end 117.82 139.9) (width 2) (layer "F.Cu") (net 31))
 (segment (start 117.82 43) (end 117.82 139.9) (width 2) (layer "B.Cu") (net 32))
 (segment (start 121.78 43) (end 121.78 139.9) (width 2) (layer "F.Cu") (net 33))
 (segment (start 121.78 43) (end 121.78 139.9) (width 2) (layer "B.Cu") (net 34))
 (segment (start 125.74 43) (end 125.74 139.9) (width 2) (layer "F.Cu") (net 35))
 (segment (start 125.74 43) (end 125.74 139.9) (width 2) (layer "B.Cu") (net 36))
 (segment (start 129.7 43) (end 129.7 139.9) (width 2) (layer "F.Cu") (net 37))
 (segment (start 129.7 43) (end 129.7 139.9) (width 2) (layer "B.Cu") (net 38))
 (segment (start 133.66 43) (end 133.66 139.9) (width 2) (layer "F.Cu") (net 39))
 (segment (start 133.66 43) (end 133.66 139.9) (width 2) (layer "B.Cu") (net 40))
 (segment (start 137.62 43) (end 137.62 139.9) (width 2) (layer "F.Cu") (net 41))
 (segment (start 137.62 43) (end 137.62 139.9) (width 2) (layer "B.Cu") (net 42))
 (segment (start 141.58 43) (end 141.58 139.9) (width 2) (layer "F.Cu") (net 43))
 (segment (start 141.58 43) (end 141.58 139.9) (width 2) (layer "B.Cu") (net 44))
 (gr_line (start 54.5 40) (end 145.5 40) (stroke (width 0.1) (type default)) (layer "Edge.Cuts"))
 (gr_arc (start 145.5 40) (mid 146.5607 40.4393) (end 147 41.5) (stroke (width 0.1) (type default)) (layer "Edge.Cuts"))
 (gr_line (start 147 41.5) (end 147 131.5) (stroke (width 0.1) (type default)) (layer "Edge.Cuts"))
 (gr_line (start 147 131.5) (end 144.5 134) (stroke (width 0.1) (type default)) (layer "Edge.Cuts"))
 (gr_line (start 144.5 134) (end 144.5 144.5) (stroke (width 0.1) (type default)) (layer "Edge.Cuts"))
 (gr_line (start 144.5 144.5) (end 144 145) (stroke (width 0.1) (type default)) (layer "Edge.Cuts"))
 (gr_line (start 144 145) (end 56 145) (stroke (width 0.1) (type default)) (layer "Edge.Cuts"))
 (gr_line (start 56 145) (end 55.5 144.5) (stroke (width 0.1) (type default)) (layer "Edge.Cuts"))
 (gr_line (start 55.5 144.5) (end 55.5 134) (stroke (width 0.1) (type default)) (layer "Edge.Cuts"))
 (gr_line (start 55.5 134) (end 53 131.5) (stroke (width 0.1) (type default)) (layer "Edge.Cuts"))
 (gr_line (start 53 131.5) (end 53 41.5) (stroke (width 0.1) (type default)) (layer "Edge.Cuts"))
 (gr_arc (start 53 41.5) (mid 53.4393 40.4393) (end 54.5 40) (stroke (width 0.1) (type default)) (layer "Edge.Cuts"))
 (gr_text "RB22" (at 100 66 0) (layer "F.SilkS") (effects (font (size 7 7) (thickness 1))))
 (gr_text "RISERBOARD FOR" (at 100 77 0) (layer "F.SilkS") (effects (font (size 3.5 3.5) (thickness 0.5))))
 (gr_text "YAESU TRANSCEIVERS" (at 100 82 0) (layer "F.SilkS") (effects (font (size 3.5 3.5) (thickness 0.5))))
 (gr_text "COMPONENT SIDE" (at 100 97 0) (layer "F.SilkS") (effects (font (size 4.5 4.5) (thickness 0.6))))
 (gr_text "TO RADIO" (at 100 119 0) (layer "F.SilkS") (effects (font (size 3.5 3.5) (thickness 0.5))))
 (gr_line (start 100 102) (end 100 114.5) (stroke (width 0.5) (type default)) (layer "F.SilkS"))
 (gr_line (start 97.5 112) (end 100 114.5) (stroke (width 0.5) (type default)) (layer "F.SilkS"))
 (gr_line (start 102.5 112) (end 100 114.5) (stroke (width 0.5) (type default)) (layer "F.SilkS")))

